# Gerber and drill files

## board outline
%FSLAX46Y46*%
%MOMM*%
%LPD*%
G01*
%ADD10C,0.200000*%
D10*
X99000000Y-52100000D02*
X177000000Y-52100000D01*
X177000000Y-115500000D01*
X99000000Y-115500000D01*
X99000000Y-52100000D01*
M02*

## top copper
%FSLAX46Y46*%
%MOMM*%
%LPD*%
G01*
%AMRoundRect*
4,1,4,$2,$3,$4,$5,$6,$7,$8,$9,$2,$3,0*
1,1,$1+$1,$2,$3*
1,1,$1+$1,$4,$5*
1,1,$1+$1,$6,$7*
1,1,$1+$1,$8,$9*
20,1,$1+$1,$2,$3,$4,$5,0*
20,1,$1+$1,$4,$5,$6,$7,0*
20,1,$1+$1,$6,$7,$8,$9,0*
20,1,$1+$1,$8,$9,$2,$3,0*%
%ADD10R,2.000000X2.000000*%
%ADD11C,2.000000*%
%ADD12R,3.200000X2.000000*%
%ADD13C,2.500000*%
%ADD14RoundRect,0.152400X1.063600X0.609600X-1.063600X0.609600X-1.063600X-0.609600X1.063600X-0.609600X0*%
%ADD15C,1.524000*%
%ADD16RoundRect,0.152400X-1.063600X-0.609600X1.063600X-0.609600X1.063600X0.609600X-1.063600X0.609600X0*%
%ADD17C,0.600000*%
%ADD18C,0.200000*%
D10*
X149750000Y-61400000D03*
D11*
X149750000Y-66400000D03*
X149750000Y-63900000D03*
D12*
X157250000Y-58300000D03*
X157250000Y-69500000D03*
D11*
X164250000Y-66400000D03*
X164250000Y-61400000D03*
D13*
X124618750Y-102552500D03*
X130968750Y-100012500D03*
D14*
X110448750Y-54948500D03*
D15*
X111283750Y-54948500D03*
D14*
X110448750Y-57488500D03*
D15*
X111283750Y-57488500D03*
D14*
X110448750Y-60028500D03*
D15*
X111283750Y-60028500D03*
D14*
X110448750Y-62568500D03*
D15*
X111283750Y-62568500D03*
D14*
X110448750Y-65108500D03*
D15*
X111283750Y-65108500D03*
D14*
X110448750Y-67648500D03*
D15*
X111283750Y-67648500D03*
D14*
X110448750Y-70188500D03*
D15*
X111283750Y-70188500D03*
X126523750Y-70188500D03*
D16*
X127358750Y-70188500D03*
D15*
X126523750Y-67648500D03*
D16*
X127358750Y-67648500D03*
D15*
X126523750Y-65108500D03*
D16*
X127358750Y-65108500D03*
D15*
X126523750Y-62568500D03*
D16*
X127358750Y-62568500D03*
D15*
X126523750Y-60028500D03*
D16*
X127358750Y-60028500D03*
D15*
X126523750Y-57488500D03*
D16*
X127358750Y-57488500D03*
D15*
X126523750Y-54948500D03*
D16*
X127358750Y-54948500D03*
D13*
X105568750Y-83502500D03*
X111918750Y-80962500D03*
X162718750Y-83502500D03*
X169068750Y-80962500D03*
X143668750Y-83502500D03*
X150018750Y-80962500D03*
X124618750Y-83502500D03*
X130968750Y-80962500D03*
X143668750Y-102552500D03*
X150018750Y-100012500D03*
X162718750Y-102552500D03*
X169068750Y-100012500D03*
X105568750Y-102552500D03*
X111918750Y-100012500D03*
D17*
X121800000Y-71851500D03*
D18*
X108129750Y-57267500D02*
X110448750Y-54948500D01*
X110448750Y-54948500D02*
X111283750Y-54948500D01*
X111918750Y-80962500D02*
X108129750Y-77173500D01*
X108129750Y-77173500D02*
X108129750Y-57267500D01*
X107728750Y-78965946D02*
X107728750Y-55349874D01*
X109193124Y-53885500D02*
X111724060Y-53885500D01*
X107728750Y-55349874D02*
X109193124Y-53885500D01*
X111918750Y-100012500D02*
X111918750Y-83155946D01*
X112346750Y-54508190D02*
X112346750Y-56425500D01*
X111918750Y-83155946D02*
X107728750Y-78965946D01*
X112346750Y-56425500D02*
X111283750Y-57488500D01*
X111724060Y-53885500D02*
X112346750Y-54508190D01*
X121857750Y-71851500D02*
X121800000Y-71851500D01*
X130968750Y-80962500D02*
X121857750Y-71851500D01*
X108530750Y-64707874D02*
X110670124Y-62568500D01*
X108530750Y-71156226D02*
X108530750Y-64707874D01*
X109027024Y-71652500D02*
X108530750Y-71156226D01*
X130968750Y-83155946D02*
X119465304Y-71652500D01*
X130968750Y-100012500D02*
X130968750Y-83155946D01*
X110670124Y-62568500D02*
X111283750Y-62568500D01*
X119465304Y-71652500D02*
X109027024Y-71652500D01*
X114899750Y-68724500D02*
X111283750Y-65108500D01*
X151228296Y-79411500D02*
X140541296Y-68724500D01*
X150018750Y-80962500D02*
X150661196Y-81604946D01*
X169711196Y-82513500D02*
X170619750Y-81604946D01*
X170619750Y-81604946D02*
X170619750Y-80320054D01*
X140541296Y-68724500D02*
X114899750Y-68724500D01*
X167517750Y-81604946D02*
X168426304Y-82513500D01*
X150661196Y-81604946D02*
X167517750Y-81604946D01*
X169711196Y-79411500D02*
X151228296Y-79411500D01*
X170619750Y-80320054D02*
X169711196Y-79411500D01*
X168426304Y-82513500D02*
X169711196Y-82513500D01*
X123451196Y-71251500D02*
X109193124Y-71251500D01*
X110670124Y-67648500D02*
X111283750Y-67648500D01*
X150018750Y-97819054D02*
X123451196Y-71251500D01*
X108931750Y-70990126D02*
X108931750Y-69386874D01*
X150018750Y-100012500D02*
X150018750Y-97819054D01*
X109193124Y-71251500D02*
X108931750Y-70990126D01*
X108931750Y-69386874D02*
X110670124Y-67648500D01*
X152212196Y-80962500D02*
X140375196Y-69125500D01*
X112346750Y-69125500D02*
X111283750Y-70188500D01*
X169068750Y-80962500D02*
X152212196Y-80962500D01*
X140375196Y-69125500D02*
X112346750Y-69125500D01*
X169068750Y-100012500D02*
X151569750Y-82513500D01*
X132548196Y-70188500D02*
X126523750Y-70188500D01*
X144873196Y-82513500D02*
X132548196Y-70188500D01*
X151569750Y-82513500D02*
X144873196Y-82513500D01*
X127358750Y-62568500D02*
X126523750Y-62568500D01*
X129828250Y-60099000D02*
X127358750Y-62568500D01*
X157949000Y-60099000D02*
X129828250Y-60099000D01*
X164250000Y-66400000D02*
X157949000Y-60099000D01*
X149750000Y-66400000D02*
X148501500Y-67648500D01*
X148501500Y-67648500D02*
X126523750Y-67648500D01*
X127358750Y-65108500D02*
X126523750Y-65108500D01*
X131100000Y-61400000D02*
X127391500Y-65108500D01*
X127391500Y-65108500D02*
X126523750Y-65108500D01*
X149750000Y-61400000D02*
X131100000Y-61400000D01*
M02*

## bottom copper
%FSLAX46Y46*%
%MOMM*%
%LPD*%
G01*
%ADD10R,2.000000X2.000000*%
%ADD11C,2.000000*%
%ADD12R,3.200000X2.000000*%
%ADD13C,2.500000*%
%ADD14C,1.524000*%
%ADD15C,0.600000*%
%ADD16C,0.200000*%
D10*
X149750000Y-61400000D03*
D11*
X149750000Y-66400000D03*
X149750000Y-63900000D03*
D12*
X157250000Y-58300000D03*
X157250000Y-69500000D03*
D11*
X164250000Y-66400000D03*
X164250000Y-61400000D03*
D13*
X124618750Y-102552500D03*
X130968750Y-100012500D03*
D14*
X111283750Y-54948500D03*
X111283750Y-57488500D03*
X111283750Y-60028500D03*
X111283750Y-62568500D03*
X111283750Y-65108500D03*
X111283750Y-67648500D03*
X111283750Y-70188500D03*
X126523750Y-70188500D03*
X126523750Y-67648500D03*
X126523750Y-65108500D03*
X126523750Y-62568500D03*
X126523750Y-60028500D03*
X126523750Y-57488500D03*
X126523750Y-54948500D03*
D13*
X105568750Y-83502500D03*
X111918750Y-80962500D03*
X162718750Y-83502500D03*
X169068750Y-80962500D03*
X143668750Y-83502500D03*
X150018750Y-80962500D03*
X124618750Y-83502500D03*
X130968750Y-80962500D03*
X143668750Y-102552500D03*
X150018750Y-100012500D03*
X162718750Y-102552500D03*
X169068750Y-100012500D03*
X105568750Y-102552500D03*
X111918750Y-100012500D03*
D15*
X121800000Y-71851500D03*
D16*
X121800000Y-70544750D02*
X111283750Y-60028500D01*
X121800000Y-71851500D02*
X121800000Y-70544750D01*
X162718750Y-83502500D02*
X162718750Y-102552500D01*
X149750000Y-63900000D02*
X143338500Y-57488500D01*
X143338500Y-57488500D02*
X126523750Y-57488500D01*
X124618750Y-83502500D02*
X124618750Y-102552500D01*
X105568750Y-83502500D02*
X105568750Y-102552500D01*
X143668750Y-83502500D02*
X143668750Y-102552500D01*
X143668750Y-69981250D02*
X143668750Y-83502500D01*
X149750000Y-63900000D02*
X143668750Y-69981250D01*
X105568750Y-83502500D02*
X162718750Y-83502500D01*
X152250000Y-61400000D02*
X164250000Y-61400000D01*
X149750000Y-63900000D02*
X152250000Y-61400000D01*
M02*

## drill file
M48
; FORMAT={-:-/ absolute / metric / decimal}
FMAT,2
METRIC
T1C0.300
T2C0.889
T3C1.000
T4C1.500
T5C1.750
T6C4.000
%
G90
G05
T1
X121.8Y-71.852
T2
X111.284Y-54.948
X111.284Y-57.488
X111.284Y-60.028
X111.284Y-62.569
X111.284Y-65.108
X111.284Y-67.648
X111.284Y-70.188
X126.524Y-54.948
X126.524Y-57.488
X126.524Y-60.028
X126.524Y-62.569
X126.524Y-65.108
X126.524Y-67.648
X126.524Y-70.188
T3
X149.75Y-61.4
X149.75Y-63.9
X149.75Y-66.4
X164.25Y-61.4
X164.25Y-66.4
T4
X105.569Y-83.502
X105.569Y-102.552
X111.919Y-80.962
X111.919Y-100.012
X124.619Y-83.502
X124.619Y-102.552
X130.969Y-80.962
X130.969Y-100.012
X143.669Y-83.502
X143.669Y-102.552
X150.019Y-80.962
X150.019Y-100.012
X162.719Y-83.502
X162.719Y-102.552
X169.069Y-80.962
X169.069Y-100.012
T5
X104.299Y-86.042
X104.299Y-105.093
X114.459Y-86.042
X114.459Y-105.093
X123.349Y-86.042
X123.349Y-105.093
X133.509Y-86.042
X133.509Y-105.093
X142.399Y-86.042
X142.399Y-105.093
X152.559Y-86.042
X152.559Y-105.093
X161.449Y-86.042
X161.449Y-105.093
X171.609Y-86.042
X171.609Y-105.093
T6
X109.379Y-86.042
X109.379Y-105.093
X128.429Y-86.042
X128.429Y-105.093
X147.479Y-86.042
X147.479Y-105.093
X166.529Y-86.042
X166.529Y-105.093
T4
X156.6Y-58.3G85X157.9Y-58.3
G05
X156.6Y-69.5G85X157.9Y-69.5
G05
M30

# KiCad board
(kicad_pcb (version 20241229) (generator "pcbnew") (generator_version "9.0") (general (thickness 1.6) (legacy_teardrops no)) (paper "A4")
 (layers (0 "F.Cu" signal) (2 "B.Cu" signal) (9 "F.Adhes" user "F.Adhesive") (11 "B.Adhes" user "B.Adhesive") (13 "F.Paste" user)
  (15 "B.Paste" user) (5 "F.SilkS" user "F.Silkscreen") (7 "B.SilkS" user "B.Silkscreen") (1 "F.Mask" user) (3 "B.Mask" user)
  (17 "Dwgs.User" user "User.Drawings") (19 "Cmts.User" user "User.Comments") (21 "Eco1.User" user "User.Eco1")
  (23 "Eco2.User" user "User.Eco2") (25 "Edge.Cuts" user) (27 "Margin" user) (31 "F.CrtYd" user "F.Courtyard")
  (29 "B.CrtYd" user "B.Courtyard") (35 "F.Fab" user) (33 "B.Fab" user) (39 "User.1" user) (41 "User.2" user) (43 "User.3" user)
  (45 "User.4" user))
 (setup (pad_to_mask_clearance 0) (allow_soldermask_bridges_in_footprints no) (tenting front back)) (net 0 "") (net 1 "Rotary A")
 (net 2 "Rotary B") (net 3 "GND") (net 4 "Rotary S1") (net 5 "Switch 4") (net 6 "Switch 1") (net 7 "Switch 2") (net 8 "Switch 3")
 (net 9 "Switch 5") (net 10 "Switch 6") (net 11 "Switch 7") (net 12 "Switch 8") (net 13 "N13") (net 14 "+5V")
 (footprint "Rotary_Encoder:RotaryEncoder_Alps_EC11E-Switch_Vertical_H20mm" (layer "F.Cu") (at 149.75 61.4)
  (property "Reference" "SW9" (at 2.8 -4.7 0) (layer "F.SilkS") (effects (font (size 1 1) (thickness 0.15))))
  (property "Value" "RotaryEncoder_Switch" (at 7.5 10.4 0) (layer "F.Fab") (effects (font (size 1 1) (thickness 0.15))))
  (pad "A" thru_hole rect (at 0 0) (size 2 2) (drill 1) (layers "*.Cu" "*.Mask") (remove_unused_layers no) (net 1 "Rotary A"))
  (pad "B" thru_hole circle (at 0 5) (size 2 2) (drill 1) (layers "*.Cu" "*.Mask") (remove_unused_layers no) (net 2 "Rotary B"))
  (pad "C" thru_hole circle (at 0 2.5) (size 2 2) (drill 1) (layers "*.Cu" "*.Mask") (remove_unused_layers no) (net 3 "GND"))
  (pad "MP" thru_hole rect (at 7.5 -3.1) (size 3.2 2) (drill oval 2.8 1.5) (layers "*.Cu" "*.Mask") (remove_unused_layers no))
  (pad "MP" thru_hole rect (at 7.5 8.1) (size 3.2 2) (drill oval 2.8 1.5) (layers "*.Cu" "*.Mask") (remove_unused_layers no))
  (pad "S1" thru_hole circle (at 14.5 5) (size 2 2) (drill 1) (layers "*.Cu" "*.Mask") (remove_unused_layers no) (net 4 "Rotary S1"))
  (pad "S2" thru_hole circle (at 14.5 0) (size 2 2) (drill 1) (layers "*.Cu" "*.Mask") (remove_unused_layers no) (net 3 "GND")))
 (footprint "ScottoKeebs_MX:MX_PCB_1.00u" (layer "F.Cu") (at 128.42875 105.0925)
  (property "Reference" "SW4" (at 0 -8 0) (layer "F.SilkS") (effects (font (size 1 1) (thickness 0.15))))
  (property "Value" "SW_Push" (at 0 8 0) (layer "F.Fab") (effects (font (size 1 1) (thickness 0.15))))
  (pad "" np_thru_hole circle (at -5.08 0) (size 1.75 1.75) (drill 1.75) (layers "*.Cu" "*.Mask"))
  (pad "" np_thru_hole circle (at 0 0) (size 4 4) (drill 4) (layers "*.Cu" "*.Mask"))
  (pad "" np_thru_hole circle (at 5.08 0) (size 1.75 1.75) (drill 1.75) (layers "*.Cu" "*.Mask"))
  (pad "1" thru_hole circle (at -3.81 -2.54) (size 2.5 2.5) (drill 1.5) (layers "*.Cu" "*.Mask") (remove_unused_layers no) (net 3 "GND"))
  (pad "2" thru_hole circle (at 2.54 -5.08) (size 2.5 2.5) (drill 1.5) (layers "*.Cu" "*.Mask") (remove_unused_layers no) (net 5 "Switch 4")))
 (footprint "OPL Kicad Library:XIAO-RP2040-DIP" (layer "F.Cu") (at 118.90375 62.5685)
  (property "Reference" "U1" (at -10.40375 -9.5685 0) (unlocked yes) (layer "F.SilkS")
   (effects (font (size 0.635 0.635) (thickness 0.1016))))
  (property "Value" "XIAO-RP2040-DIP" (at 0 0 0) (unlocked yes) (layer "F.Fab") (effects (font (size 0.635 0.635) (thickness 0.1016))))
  (pad "1" smd roundrect (at -8.455 -7.62 180) (size 2.432 1.524) (layers "F.Cu" "F.Mask") (roundrect_rratio 0.1) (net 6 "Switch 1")
   (thermal_bridge_angle 45))
  (pad "1" thru_hole circle (at -7.62 -7.62 180) (size 1.524 1.524) (drill 0.889) (layers "*.Cu" "*.Mask") (remove_unused_layers no)
   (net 6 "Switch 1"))
  (pad "2" smd roundrect (at -8.455 -5.08 180) (size 2.432 1.524) (layers "F.Cu" "F.Mask") (roundrect_rratio 0.1) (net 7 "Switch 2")
   (thermal_bridge_angle 45))
  (pad "2" thru_hole circle (at -7.62 -5.08 180) (size 1.524 1.524) (drill 0.889) (layers "*.Cu" "*.Mask") (remove_unused_layers no)
   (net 7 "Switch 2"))
  (pad "3" smd roundrect (at -8.455 -2.54 180) (size 2.432 1.524) (layers "F.Cu" "F.Mask") (roundrect_rratio 0.1) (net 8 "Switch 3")
   (thermal_bridge_angle 45))
  (pad "3" thru_hole circle (at -7.62 -2.54 180) (size 1.524 1.524) (drill 0.889) (layers "*.Cu" "*.Mask") (remove_unused_layers no)
   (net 8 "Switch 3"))
  (pad "4" smd roundrect (at -8.455 0 180) (size 2.432 1.524) (layers "F.Cu" "F.Mask") (roundrect_rratio 0.1) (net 5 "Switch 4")
   (thermal_bridge_angle 45))
  (pad "4" thru_hole circle (at -7.62 0 180) (size 1.524 1.524) (drill 0.889) (layers "*.Cu" "*.Mask") (remove_unused_layers no)
   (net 5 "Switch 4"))
  (pad "5" smd roundrect (at -8.455 2.54 180) (size 2.432 1.524) (layers "F.Cu" "F.Mask") (roundrect_rratio 0.1) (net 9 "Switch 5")
   (thermal_bridge_angle 45))
  (pad "5" thru_hole circle (at -7.62 2.54 180) (size 1.524 1.524) (drill 0.889) (layers "*.Cu" "*.Mask") (remove_unused_layers no)
   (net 9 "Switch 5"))
  (pad "6" smd roundrect (at -8.455 5.08 180) (size 2.432 1.524) (layers "F.Cu" "F.Mask") (roundrect_rratio 0.1) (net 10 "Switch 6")
   (thermal_bridge_angle 45))
  (pad "6" thru_hole circle (at -7.62 5.08 180) (size 1.524 1.524) (drill 0.889) (layers "*.Cu" "*.Mask") (remove_unused_layers no)
   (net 10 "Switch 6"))
  (pad "7" smd roundrect (at -8.455 7.62 180) (size 2.432 1.524) (layers "F.Cu" "F.Mask") (roundrect_rratio 0.1) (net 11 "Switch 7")
   (thermal_bridge_angle 45))
  (pad "7" thru_hole circle (at -7.62 7.62 180) (size 1.524 1.524) (drill 0.889) (layers "*.Cu" "*.Mask") (remove_unused_layers no)
   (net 11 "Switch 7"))
  (pad "8" thru_hole circle (at 7.62 7.62) (size 1.524 1.524) (drill 0.889) (layers "*.Cu" "*.Mask") (remove_unused_layers no)
   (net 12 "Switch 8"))
  (pad "8" smd roundrect (at 8.455 7.62) (size 2.432 1.524) (layers "F.Cu" "F.Mask") (roundrect_rratio 0.1) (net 12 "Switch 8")
   (thermal_bridge_angle 45))
  (pad "9" thru_hole circle (at 7.62 5.08) (size 1.524 1.524) (drill 0.889) (layers "*.Cu" "*.Mask") (remove_unused_layers no)
   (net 2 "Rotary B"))
  (pad "9" smd roundrect (at 8.455 5.08) (size 2.432 1.524) (layers "F.Cu" "F.Mask") (roundrect_rratio 0.1) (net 2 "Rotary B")
   (thermal_bridge_angle 45))
  (pad "10" thru_hole circle (at 7.62 2.54) (size 1.524 1.524) (drill 0.889) (layers "*.Cu" "*.Mask") (remove_unused_layers no)
   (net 1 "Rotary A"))
  (pad "10" smd roundrect (at 8.455 2.54) (size 2.432 1.524) (layers "F.Cu" "F.Mask") (roundrect_rratio 0.1) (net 1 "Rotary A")
   (thermal_bridge_angle 45))
  (pad "11" thru_hole circle (at 7.62 0) (size 1.524 1.524) (drill 0.889) (layers "*.Cu" "*.Mask") (remove_unused_layers no)
   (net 4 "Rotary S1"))
  (pad "11" smd roundrect (at 8.455 0) (size 2.432 1.524) (layers "F.Cu" "F.Mask") (roundrect_rratio 0.1) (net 4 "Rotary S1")
   (thermal_bridge_angle 45))
  (pad "12" thru_hole circle (at 7.62 -2.54) (size 1.524 1.524) (drill 0.889) (layers "*.Cu" "*.Mask") (remove_unused_layers no)
   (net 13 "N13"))
  (pad "12" smd roundrect (at 8.455 -2.54) (size 2.432 1.524) (layers "F.Cu" "F.Mask") (roundrect_rratio 0.1) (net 13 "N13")
   (thermal_bridge_angle 45))
  (pad "13" thru_hole circle (at 7.62 -5.08) (size 1.524 1.524) (drill 0.889) (layers "*.Cu" "*.Mask") (remove_unused_layers no)
   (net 3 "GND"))
  (pad "13" smd roundrect (at 8.455 -5.08) (size 2.432 1.524) (layers "F.Cu" "F.Mask") (roundrect_rratio 0.1) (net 3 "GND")
   (thermal_bridge_angle 45))
  (pad "14" thru_hole circle (at 7.62 -7.62) (size 1.524 1.524) (drill 0.889) (layers "*.Cu" "*.Mask") (remove_unused_layers no)
   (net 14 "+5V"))
  (pad "14" smd roundrect (at 8.455 -7.62) (size 2.432 1.524) (layers "F.Cu" "F.Mask") (roundrect_rratio 0.1) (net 14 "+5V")
   (thermal_bridge_angle 45)))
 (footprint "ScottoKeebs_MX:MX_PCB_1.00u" (layer "F.Cu") (at 109.37875 86.0425)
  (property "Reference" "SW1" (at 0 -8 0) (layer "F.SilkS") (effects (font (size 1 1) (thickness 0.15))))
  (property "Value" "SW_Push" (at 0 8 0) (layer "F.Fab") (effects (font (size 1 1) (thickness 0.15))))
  (pad "" np_thru_hole circle (at -5.08 0) (size 1.75 1.75) (drill 1.75) (layers "*.Cu" "*.Mask"))
  (pad "" np_thru_hole circle (at 0 0) (size 4 4) (drill 4) (layers "*.Cu" "*.Mask"))
  (pad "" np_thru_hole circle (at 5.08 0) (size 1.75 1.75) (drill 1.75) (layers "*.Cu" "*.Mask"))
  (pad "1" thru_hole circle (at -3.81 -2.54) (size 2.5 2.5) (drill 1.5) (layers "*.Cu" "*.Mask") (remove_unused_layers no) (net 3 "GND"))
  (pad "2" thru_hole circle (at 2.54 -5.08) (size 2.5 2.5) (drill 1.5) (layers "*.Cu" "*.Mask") (remove_unused_layers no) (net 6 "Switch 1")))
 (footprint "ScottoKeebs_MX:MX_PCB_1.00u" (layer "F.Cu") (at 166.52875 86.0425)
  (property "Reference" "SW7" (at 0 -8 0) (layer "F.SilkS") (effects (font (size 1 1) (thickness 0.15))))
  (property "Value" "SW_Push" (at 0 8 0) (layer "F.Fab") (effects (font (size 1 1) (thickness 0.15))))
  (pad "" np_thru_hole circle (at -5.08 0) (size 1.75 1.75) (drill 1.75) (layers "*.Cu" "*.Mask"))
  (pad "" np_thru_hole circle (at 0 0) (size 4 4) (drill 4) (layers "*.Cu" "*.Mask"))
  (pad "" np_thru_hole circle (at 5.08 0) (size 1.75 1.75) (drill 1.75) (layers "*.Cu" "*.Mask"))
  (pad "1" thru_hole circle (at -3.81 -2.54) (size 2.5 2.5) (drill 1.5) (layers "*.Cu" "*.Mask") (remove_unused_layers no) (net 3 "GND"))
  (pad "2" thru_hole circle (at 2.54 -5.08) (size 2.5 2.5) (drill 1.5) (layers "*.Cu" "*.Mask") (remove_unused_layers no)
   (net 11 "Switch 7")))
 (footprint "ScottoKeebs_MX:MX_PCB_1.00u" (layer "F.Cu") (at 147.47875 86.0425)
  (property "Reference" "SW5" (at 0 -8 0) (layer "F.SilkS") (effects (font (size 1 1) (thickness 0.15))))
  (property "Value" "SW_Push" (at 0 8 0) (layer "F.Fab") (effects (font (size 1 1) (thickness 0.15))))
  (pad "" np_thru_hole circle (at -5.08 0) (size 1.75 1.75) (drill 1.75) (layers "*.Cu" "*.Mask"))
  (pad "" np_thru_hole circle (at 0 0) (size 4 4) (drill 4) (layers "*.Cu" "*.Mask"))
  (pad "" np_thru_hole circle (at 5.08 0) (size 1.75 1.75) (drill 1.75) (layers "*.Cu" "*.Mask"))
  (pad "1" thru_hole circle (at -3.81 -2.54) (size 2.5 2.5) (drill 1.5) (layers "*.Cu" "*.Mask") (remove_unused_layers no) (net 3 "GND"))
  (pad "2" thru_hole circle (at 2.54 -5.08) (size 2.5 2.5) (drill 1.5) (layers "*.Cu" "*.Mask") (remove_unused_layers no) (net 9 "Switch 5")))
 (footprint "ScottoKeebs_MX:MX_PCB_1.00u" (layer "F.Cu") (at 128.42875 86.0425)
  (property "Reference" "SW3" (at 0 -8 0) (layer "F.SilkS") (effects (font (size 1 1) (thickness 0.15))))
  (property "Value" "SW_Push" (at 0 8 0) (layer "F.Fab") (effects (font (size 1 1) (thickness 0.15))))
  (pad "" np_thru_hole circle (at -5.08 0) (size 1.75 1.75) (drill 1.75) (layers "*.Cu" "*.Mask"))
  (pad "" np_thru_hole circle (at 0 0) (size 4 4) (drill 4) (layers "*.Cu" "*.Mask"))
  (pad "" np_thru_hole circle (at 5.08 0) (size 1.75 1.75) (drill 1.75) (layers "*.Cu" "*.Mask"))
  (pad "1" thru_hole circle (at -3.81 -2.54) (size 2.5 2.5) (drill 1.5) (layers "*.Cu" "*.Mask") (remove_unused_layers no) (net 3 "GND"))
  (pad "2" thru_hole circle (at 2.54 -5.08) (size 2.5 2.5) (drill 1.5) (layers "*.Cu" "*.Mask") (remove_unused_layers no) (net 8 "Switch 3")))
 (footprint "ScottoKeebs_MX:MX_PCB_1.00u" (layer "F.Cu") (at 147.47875 105.0925)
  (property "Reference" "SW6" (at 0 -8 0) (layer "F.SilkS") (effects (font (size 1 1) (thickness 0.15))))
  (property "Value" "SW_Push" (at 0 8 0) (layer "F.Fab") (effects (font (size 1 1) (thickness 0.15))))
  (pad "" np_thru_hole circle (at -5.08 0) (size 1.75 1.75) (drill 1.75) (layers "*.Cu" "*.Mask"))
  (pad "" np_thru_hole circle (at 0 0) (size 4 4) (drill 4) (layers "*.Cu" "*.Mask"))
  (pad "" np_thru_hole circle (at 5.08 0) (size 1.75 1.75) (drill 1.75) (layers "*.Cu" "*.Mask"))
  (pad "1" thru_hole circle (at -3.81 -2.54) (size 2.5 2.5) (drill 1.5) (layers "*.Cu" "*.Mask") (remove_unused_layers no) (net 3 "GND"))
  (pad "2" thru_hole circle (at 2.54 -5.08) (size 2.5 2.5) (drill 1.5) (layers "*.Cu" "*.Mask") (remove_unused_layers no)
   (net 10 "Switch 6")))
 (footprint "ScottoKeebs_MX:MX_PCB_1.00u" (layer "F.Cu") (at 166.52875 105.0925)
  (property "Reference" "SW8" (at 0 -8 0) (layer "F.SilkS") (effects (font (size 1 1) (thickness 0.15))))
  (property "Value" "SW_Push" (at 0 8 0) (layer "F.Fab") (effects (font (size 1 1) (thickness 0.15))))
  (pad "" np_thru_hole circle (at -5.08 0) (size 1.75 1.75) (drill 1.75) (layers "*.Cu" "*.Mask"))
  (pad "" np_thru_hole circle (at 0 0) (size 4 4) (drill 4) (layers "*.Cu" "*.Mask"))
  (pad "" np_thru_hole circle (at 5.08 0) (size 1.75 1.75) (drill 1.75) (layers "*.Cu" "*.Mask"))
  (pad "1" thru_hole circle (at -3.81 -2.54) (size 2.5 2.5) (drill 1.5) (layers "*.Cu" "*.Mask") (remove_unused_layers no) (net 3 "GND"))
  (pad "2" thru_hole circle (at 2.54 -5.08) (size 2.5 2.5) (drill 1.5) (layers "*.Cu" "*.Mask") (remove_unused_layers no)
   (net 12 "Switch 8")))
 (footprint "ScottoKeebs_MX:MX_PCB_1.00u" (layer "F.Cu") (at 109.37875 105.0925)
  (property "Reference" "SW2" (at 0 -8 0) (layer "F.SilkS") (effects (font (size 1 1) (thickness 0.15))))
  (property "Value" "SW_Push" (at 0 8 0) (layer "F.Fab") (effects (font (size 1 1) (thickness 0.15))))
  (pad "" np_thru_hole circle (at -5.08 0) (size 1.75 1.75) (drill 1.75) (layers "*.Cu" "*.Mask"))
  (pad "" np_thru_hole circle (at 0 0) (size 4 4) (drill 4) (layers "*.Cu" "*.Mask"))
  (pad "" np_thru_hole circle (at 5.08 0) (size 1.75 1.75) (drill 1.75) (layers "*.Cu" "*.Mask"))
  (pad "1" thru_hole circle (at -3.81 -2.54) (size 2.5 2.5) (drill 1.5) (layers "*.Cu" "*.Mask") (remove_unused_layers no) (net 3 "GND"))
  (pad "2" thru_hole circle (at 2.54 -5.08) (size 2.5 2.5) (drill 1.5) (layers "*.Cu" "*.Mask") (remove_unused_layers no) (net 7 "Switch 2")))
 (gr_rect (start 99 52.1) (end 177 115.5) (stroke (width 0.2) (type solid)) (fill no) (layer "Edge.Cuts"))
 (segment (start 108.12975 57.2675) (end 110.44875 54.9485) (width 0.2) (layer "F.Cu") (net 6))
 (segment (start 110.44875 54.9485) (end 111.28375 54.9485) (width 0.2) (layer "F.Cu") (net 6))
 (segment (start 111.91875 80.9625) (end 108.12975 77.1735) (width 0.2) (layer "F.Cu") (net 6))
 (segment (start 108.12975 77.1735) (end 108.12975 57.2675) (width 0.2) (layer "F.Cu") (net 6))
 (segment (start 107.72875 78.965946) (end 107.72875 55.349874) (width 0.2) (layer "F.Cu") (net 7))
 (segment (start 109.193124 53.8855) (end 111.72406 53.8855) (width 0.2) (layer "F.Cu") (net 7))
 (segment (start 107.72875 55.349874) (end 109.193124 53.8855) (width 0.2) (layer "F.Cu") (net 7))
 (segment (start 111.91875 100.0125) (end 111.91875 83.155946) (width 0.2) (layer "F.Cu") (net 7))
 (segment (start 112.34675 54.50819) (end 112.34675 56.4255) (width 0.2) (layer "F.Cu") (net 7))
 (segment (start 111.91875 83.155946) (end 107.72875 78.965946) (width 0.2) (layer "F.Cu") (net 7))
 (segment (start 112.34675 56.4255) (end 111.28375 57.4885) (width 0.2) (layer "F.Cu") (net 7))
 (segment (start 111.72406 53.8855) (end 112.34675 54.50819) (width 0.2) (layer "F.Cu") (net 7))
 (segment (start 121.85775 71.8515) (end 121.8 71.8515) (width 0.2) (layer "F.Cu") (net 8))
 (segment (start 130.96875 80.9625) (end 121.85775 71.8515) (width 0.2) (layer "F.Cu") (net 8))
 (via (at 121.8 71.8515) (size 0.6) (drill 0.3) (layers "F.Cu" "B.Cu") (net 8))
 (segment (start 121.8 70.54475) (end 111.28375 60.0285) (width 0.2) (layer "B.Cu") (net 8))
 (segment (start 121.8 71.8515) (end 121.8 70.54475) (width 0.2) (layer "B.Cu") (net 8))
 (segment (start 108.53075 64.707874) (end 110.670124 62.5685) (width 0.2) (layer "F.Cu") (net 5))
 (segment (start 108.53075 71.156226) (end 108.53075 64.707874) (width 0.2) (layer "F.Cu") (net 5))
 (segment (start 109.027024 71.6525) (end 108.53075 71.156226) (width 0.2) (layer "F.Cu") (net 5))
 (segment (start 130.96875 83.155946) (end 119.465304 71.6525) (width 0.2) (layer "F.Cu") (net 5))
 (segment (start 130.96875 100.0125) (end 130.96875 83.155946) (width 0.2) (layer "F.Cu") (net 5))
 (segment (start 110.670124 62.5685) (end 111.28375 62.5685) (width 0.2) (layer "F.Cu") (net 5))
 (segment (start 119.465304 71.6525) (end 109.027024 71.6525) (width 0.2) (layer "F.Cu") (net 5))
 (segment (start 114.89975 68.7245) (end 111.28375 65.1085) (width 0.2) (layer "F.Cu") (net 9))
 (segment (start 151.228296 79.4115) (end 140.541296 68.7245) (width 0.2) (layer "F.Cu") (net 9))
 (segment (start 150.01875 80.9625) (end 150.661196 81.604946) (width 0.2) (layer "F.Cu") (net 9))
 (segment (start 169.711196 82.5135) (end 170.61975 81.604946) (width 0.2) (layer "F.Cu") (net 9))
 (segment (start 170.61975 81.604946) (end 170.61975 80.320054) (width 0.2) (layer "F.Cu") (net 9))
 (segment (start 140.541296 68.7245) (end 114.89975 68.7245) (width 0.2) (layer "F.Cu") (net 9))
 (segment (start 167.51775 81.604946) (end 168.426304 82.5135) (width 0.2) (layer "F.Cu") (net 9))
 (segment (start 150.661196 81.604946) (end 167.51775 81.604946) (width 0.2) (layer "F.Cu") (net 9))
 (segment (start 169.711196 79.4115) (end 151.228296 79.4115) (width 0.2) (layer "F.Cu") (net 9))
 (segment (start 170.61975 80.320054) (end 169.711196 79.4115) (width 0.2) (layer "F.Cu") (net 9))
 (segment (start 168.426304 82.5135) (end 169.711196 82.5135) (width 0.2) (layer "F.Cu") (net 9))
 (segment (start 123.451196 71.2515) (end 109.193124 71.2515) (width 0.2) (layer "F.Cu") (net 10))
 (segment (start 110.670124 67.6485) (end 111.28375 67.6485) (width 0.2) (layer "F.Cu") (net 10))
 (segment (start 150.01875 97.819054) (end 123.451196 71.2515) (width 0.2) (layer "F.Cu") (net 10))
 (segment (start 108.93175 70.990126) (end 108.93175 69.386874) (width 0.2) (layer "F.Cu") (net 10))
 (segment (start 150.01875 100.0125) (end 150.01875 97.819054) (width 0.2) (layer "F.Cu") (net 10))
 (segment (start 109.193124 71.2515) (end 108.93175 70.990126) (width 0.2) (layer "F.Cu") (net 10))
 (segment (start 108.93175 69.386874) (end 110.670124 67.6485) (width 0.2) (layer "F.Cu") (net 10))
 (segment (start 152.212196 80.9625) (end 140.375196 69.1255) (width 0.2) (layer "F.Cu") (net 11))
 (segment (start 112.34675 69.1255) (end 111.28375 70.1885) (width 0.2) (layer "F.Cu") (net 11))
 (segment (start 169.06875 80.9625) (end 152.212196 80.9625) (width 0.2) (layer "F.Cu") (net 11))
 (segment (start 140.375196 69.1255) (end 112.34675 69.1255) (width 0.2) (layer "F.Cu") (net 11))
 (segment (start 169.06875 100.0125) (end 151.56975 82.5135) (width 0.2) (layer "F.Cu") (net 12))
 (segment (start 132.548196 70.1885) (end 126.52375 70.1885) (width 0.2) (layer "F.Cu") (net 12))
 (segment (start 144.873196 82.5135) (end 132.548196 70.1885) (width 0.2) (layer "F.Cu") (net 12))
 (segment (start 151.56975 82.5135) (end 144.873196 82.5135) (width 0.2) (layer "F.Cu") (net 12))
 (segment (start 127.35875 62.5685) (end 126.52375 62.5685) (width 0.2) (layer "F.Cu") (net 4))
 (segment (start 129.82825 60.099) (end 127.35875 62.5685) (width 0.2) (layer "F.Cu") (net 4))
 (segment (start 157.949 60.099) (end 129.82825 60.099) (width 0.2) (layer "F.Cu") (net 4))
 (segment (start 164.25 66.4) (end 157.949 60.099) (width 0.2) (layer "F.Cu") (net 4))
 (segment (start 149.75 66.4) (end 148.5015 67.6485) (width 0.2) (layer "F.Cu") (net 2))
 (segment (start 148.5015 67.6485) (end 126.52375 67.6485) (width 0.2) (layer "F.Cu") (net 2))
 (segment (start 127.35875 65.1085) (end 126.52375 65.1085) (width 0.2) (layer "F.Cu") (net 1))
 (segment (start 131.1 61.4) (end 127.3915 65.1085) (width 0.2) (layer "F.Cu") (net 1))
 (segment (start 127.3915 65.1085) (end 126.52375 65.1085) (width 0.2) (layer "F.Cu") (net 1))
 (segment (start 149.75 61.4) (end 131.1 61.4) (width 0.2) (layer "F.Cu") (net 1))
 (segment (start 162.71875 83.5025) (end 162.71875 102.5525) (width 0.2) (layer "B.Cu") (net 3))
 (segment (start 149.75 63.9) (end 143.3385 57.4885) (width 0.2) (layer "B.Cu") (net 3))
 (segment (start 143.3385 57.4885) (end 126.52375 57.4885) (width 0.2) (layer "B.Cu") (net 3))
 (segment (start 124.61875 83.5025) (end 124.61875 102.5525) (width 0.2) (layer "B.Cu") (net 3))
 (segment (start 105.56875 83.5025) (end 105.56875 102.5525) (width 0.2) (layer "B.Cu") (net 3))
 (segment (start 143.66875 83.5025) (end 143.66875 102.5525) (width 0.2) (layer "B.Cu") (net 3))
 (segment (start 143.66875 69.98125) (end 143.66875 83.5025) (width 0.2) (layer "B.Cu") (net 3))
 (segment (start 149.75 63.9) (end 143.66875 69.98125) (width 0.2) (layer "B.Cu") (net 3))
 (segment (start 105.56875 83.5025) (end 162.71875 83.5025) (width 0.2) (layer "B.Cu") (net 3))
 (segment (start 152.25 61.4) (end 164.25 61.4) (width 0.2) (layer "B.Cu") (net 3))
 (segment (start 149.75 63.9) (end 152.25 61.4) (width 0.2) (layer "B.Cu") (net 3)))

